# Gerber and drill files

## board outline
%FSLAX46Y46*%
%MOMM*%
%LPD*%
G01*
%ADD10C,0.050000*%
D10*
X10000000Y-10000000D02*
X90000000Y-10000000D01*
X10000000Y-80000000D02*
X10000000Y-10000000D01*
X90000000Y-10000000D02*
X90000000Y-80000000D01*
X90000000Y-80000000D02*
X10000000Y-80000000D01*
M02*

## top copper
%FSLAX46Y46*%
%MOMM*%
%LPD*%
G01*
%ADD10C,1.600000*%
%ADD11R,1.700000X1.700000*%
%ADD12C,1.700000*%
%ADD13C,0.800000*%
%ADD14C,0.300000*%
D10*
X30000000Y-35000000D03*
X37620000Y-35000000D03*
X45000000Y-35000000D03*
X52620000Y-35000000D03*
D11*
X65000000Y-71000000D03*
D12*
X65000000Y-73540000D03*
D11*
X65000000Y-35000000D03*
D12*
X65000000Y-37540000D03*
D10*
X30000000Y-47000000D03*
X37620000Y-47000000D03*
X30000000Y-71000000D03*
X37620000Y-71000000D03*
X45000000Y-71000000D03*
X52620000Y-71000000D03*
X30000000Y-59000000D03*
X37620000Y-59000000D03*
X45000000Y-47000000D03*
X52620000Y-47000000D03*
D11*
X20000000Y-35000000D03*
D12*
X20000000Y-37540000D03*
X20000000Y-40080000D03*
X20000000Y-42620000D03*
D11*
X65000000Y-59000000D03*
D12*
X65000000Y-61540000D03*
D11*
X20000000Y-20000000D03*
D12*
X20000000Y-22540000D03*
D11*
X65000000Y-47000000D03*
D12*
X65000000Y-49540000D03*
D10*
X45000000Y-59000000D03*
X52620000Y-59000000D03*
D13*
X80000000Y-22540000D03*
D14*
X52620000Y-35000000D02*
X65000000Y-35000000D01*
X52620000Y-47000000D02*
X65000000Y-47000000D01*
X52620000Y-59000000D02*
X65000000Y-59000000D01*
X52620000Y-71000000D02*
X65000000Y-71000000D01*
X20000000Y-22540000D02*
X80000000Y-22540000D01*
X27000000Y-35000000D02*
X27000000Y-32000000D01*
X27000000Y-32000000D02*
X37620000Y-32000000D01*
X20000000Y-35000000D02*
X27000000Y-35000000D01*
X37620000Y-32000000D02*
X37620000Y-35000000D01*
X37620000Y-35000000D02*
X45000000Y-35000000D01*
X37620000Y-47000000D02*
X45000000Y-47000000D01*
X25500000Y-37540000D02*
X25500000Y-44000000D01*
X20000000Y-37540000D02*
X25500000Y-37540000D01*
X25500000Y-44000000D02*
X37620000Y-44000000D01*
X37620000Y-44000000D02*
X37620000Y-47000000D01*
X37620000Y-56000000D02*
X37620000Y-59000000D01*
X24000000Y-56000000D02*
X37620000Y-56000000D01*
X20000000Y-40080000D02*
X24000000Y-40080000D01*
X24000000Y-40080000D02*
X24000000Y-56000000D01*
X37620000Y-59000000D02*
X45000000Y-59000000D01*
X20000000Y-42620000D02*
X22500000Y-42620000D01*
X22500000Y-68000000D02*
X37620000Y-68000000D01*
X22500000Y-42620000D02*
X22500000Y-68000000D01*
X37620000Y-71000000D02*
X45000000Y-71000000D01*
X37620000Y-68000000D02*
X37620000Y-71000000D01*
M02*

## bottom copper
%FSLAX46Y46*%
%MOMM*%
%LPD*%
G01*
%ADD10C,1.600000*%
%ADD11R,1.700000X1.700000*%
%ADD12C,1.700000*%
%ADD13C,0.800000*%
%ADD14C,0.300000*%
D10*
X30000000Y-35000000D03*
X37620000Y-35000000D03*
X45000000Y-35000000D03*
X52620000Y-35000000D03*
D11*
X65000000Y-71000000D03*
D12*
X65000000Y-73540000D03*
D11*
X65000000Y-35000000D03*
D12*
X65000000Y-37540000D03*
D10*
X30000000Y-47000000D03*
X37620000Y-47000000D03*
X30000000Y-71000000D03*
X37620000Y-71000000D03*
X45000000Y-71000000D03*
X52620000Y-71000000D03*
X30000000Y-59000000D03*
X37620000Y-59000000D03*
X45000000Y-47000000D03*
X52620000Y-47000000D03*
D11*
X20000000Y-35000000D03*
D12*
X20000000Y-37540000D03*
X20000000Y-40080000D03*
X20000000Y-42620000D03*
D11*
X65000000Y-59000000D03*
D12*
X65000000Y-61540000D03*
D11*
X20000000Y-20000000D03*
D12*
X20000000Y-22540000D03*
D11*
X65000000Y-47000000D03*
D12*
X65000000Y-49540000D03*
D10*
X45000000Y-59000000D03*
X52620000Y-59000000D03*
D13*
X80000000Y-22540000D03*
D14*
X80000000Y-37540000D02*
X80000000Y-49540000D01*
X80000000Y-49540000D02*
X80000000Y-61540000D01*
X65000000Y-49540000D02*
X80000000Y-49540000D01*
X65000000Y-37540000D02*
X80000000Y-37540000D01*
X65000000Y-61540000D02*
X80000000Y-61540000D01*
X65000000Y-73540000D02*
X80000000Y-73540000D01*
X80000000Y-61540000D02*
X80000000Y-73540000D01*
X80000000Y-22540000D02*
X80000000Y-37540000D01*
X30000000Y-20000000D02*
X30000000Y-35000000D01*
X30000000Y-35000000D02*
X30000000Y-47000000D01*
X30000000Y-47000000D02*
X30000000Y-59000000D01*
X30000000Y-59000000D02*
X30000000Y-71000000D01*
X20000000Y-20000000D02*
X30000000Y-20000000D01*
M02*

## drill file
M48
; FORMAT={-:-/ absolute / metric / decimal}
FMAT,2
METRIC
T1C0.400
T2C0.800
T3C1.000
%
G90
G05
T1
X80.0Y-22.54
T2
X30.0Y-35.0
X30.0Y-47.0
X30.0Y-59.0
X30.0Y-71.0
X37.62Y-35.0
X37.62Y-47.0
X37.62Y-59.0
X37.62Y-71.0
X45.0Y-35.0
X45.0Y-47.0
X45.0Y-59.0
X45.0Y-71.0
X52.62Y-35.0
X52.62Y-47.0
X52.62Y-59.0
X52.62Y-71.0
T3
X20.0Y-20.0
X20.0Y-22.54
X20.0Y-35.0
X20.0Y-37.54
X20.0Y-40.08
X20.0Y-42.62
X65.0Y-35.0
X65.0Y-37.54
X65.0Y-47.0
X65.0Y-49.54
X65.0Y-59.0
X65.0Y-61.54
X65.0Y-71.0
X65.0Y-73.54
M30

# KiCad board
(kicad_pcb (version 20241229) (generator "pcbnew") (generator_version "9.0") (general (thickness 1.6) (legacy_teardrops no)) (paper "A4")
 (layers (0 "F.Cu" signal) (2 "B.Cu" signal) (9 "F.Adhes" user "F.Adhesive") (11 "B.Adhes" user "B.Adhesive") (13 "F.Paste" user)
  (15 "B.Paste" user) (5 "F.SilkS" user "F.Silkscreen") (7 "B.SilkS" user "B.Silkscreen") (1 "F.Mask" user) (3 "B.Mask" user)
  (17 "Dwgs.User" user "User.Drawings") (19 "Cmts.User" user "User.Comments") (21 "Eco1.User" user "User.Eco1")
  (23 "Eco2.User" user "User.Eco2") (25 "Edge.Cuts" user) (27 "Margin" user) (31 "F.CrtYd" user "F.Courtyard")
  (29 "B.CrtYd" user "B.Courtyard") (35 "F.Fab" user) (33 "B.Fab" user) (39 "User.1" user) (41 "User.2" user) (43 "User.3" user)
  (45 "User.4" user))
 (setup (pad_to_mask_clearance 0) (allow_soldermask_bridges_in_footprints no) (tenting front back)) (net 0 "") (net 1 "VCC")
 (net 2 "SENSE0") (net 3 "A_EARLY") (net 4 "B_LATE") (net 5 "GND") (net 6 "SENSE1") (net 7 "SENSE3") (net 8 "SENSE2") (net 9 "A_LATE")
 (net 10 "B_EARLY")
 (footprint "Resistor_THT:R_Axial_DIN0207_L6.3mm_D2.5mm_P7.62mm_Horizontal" (layer "F.Cu") (at 30 35)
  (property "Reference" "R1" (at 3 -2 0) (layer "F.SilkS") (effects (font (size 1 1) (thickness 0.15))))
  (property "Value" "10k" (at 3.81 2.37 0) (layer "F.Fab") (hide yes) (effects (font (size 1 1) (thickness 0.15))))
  (pad "1" thru_hole circle (at 0 0) (size 1.6 1.6) (drill 0.8) (layers "*.Cu" "*.Mask") (remove_unused_layers no) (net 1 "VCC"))
  (pad "2" thru_hole circle (at 7.62 0) (size 1.6 1.6) (drill 0.8) (layers "*.Cu" "*.Mask") (remove_unused_layers no) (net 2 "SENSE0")))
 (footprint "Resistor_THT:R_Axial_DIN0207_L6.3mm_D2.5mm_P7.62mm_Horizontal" (layer "F.Cu") (at 45 35)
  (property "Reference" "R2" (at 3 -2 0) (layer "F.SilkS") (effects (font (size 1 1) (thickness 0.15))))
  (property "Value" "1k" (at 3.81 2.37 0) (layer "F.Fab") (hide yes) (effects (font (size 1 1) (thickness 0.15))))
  (pad "1" thru_hole circle (at 0 0) (size 1.6 1.6) (drill 0.8) (layers "*.Cu" "*.Mask") (remove_unused_layers no) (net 2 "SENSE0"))
  (pad "2" thru_hole circle (at 7.62 0) (size 1.6 1.6) (drill 0.8) (layers "*.Cu" "*.Mask") (remove_unused_layers no) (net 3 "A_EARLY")))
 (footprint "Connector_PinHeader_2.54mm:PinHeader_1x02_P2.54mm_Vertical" (layer "F.Cu") (at 65 71)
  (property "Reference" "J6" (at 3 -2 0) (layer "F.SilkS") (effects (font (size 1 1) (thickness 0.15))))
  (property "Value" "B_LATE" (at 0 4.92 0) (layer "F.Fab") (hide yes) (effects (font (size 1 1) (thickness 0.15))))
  (pad "1" thru_hole rect (at 0 0) (size 1.7 1.7) (drill 1) (layers "*.Cu" "*.Mask") (remove_unused_layers no) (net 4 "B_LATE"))
  (pad "2" thru_hole circle (at 0 2.54) (size 1.7 1.7) (drill 1) (layers "*.Cu" "*.Mask") (remove_unused_layers no) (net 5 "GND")))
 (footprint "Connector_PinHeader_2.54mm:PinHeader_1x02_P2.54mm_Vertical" (layer "F.Cu") (at 65 35)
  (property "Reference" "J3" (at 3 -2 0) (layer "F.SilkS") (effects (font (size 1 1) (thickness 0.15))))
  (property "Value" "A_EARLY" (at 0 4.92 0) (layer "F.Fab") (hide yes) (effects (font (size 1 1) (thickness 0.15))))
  (pad "1" thru_hole rect (at 0 0) (size 1.7 1.7) (drill 1) (layers "*.Cu" "*.Mask") (remove_unused_layers no) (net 3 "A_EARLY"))
  (pad "2" thru_hole circle (at 0 2.54) (size 1.7 1.7) (drill 1) (layers "*.Cu" "*.Mask") (remove_unused_layers no) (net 5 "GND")))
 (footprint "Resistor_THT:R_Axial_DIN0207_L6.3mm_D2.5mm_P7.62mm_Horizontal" (layer "F.Cu") (at 30 47)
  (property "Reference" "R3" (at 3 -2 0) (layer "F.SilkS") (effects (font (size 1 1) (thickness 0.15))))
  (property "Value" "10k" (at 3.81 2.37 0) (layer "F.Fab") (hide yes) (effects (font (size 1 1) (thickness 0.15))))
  (pad "1" thru_hole circle (at 0 0) (size 1.6 1.6) (drill 0.8) (layers "*.Cu" "*.Mask") (remove_unused_layers no) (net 1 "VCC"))
  (pad "2" thru_hole circle (at 7.62 0) (size 1.6 1.6) (drill 0.8) (layers "*.Cu" "*.Mask") (remove_unused_layers no) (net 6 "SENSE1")))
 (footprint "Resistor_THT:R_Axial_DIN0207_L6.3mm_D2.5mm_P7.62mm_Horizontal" (layer "F.Cu") (at 30 71)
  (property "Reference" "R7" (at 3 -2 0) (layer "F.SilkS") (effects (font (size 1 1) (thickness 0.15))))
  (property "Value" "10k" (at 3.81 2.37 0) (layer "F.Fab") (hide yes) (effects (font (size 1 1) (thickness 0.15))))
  (pad "1" thru_hole circle (at 0 0) (size 1.6 1.6) (drill 0.8) (layers "*.Cu" "*.Mask") (remove_unused_layers no) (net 1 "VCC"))
  (pad "2" thru_hole circle (at 7.62 0) (size 1.6 1.6) (drill 0.8) (layers "*.Cu" "*.Mask") (remove_unused_layers no) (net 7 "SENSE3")))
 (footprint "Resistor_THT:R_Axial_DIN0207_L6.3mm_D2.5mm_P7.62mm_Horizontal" (layer "F.Cu") (at 45 71)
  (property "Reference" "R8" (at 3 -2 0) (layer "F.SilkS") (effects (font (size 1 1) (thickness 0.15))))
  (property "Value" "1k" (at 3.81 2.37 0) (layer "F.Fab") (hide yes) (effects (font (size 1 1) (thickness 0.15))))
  (pad "1" thru_hole circle (at 0 0) (size 1.6 1.6) (drill 0.8) (layers "*.Cu" "*.Mask") (remove_unused_layers no) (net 7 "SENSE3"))
  (pad "2" thru_hole circle (at 7.62 0) (size 1.6 1.6) (drill 0.8) (layers "*.Cu" "*.Mask") (remove_unused_layers no) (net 4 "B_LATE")))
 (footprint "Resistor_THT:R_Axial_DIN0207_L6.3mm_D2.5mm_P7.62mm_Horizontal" (layer "F.Cu") (at 30 59)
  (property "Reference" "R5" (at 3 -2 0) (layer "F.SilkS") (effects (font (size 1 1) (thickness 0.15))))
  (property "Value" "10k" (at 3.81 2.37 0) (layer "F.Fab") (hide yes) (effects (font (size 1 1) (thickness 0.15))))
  (pad "1" thru_hole circle (at 0 0) (size 1.6 1.6) (drill 0.8) (layers "*.Cu" "*.Mask") (remove_unused_layers no) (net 1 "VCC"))
  (pad "2" thru_hole circle (at 7.62 0) (size 1.6 1.6) (drill 0.8) (layers "*.Cu" "*.Mask") (remove_unused_layers no) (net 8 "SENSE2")))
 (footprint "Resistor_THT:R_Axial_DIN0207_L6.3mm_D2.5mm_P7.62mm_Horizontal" (layer "F.Cu") (at 45 47)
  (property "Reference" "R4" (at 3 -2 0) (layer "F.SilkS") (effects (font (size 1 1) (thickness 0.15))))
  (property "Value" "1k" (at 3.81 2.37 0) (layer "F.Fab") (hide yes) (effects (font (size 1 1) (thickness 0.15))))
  (pad "1" thru_hole circle (at 0 0) (size 1.6 1.6) (drill 0.8) (layers "*.Cu" "*.Mask") (remove_unused_layers no) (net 6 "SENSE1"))
  (pad "2" thru_hole circle (at 7.62 0) (size 1.6 1.6) (drill 0.8) (layers "*.Cu" "*.Mask") (remove_unused_layers no) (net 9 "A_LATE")))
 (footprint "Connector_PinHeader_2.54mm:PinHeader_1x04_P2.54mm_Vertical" (layer "F.Cu") (at 20 35)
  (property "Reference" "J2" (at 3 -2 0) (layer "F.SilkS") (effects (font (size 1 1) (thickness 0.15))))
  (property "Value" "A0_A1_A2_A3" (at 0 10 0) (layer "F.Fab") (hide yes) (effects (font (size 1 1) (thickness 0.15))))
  (pad "1" thru_hole rect (at 0 0) (size 1.7 1.7) (drill 1) (layers "*.Cu" "*.Mask") (remove_unused_layers no) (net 2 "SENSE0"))
  (pad "2" thru_hole circle (at 0 2.54) (size 1.7 1.7) (drill 1) (layers "*.Cu" "*.Mask") (remove_unused_layers no) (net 6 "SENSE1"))
  (pad "3" thru_hole circle (at 0 5.08) (size 1.7 1.7) (drill 1) (layers "*.Cu" "*.Mask") (remove_unused_layers no) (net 8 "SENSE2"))
  (pad "4" thru_hole circle (at 0 7.62) (size 1.7 1.7) (drill 1) (layers "*.Cu" "*.Mask") (remove_unused_layers no) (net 7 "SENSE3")))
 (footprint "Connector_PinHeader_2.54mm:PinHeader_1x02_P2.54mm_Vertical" (layer "F.Cu") (at 65 59)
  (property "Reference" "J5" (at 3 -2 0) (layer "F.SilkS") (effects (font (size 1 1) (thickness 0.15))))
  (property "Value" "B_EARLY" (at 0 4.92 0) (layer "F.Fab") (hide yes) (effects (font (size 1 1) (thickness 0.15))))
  (pad "1" thru_hole rect (at 0 0) (size 1.7 1.7) (drill 1) (layers "*.Cu" "*.Mask") (remove_unused_layers no) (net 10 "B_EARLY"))
  (pad "2" thru_hole circle (at 0 2.54) (size 1.7 1.7) (drill 1) (layers "*.Cu" "*.Mask") (remove_unused_layers no) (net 5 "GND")))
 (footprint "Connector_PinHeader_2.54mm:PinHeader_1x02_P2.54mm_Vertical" (layer "F.Cu") (at 20 20)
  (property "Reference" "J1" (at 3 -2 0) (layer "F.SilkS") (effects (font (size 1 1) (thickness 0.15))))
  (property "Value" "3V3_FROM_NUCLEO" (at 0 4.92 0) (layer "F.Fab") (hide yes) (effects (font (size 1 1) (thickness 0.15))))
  (pad "1" thru_hole rect (at 0 0) (size 1.7 1.7) (drill 1) (layers "*.Cu" "*.Mask") (remove_unused_layers no) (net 1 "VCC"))
  (pad "2" thru_hole circle (at 0 2.54) (size 1.7 1.7) (drill 1) (layers "*.Cu" "*.Mask") (remove_unused_layers no) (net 5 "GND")))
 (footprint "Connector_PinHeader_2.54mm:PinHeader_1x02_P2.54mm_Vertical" (layer "F.Cu") (at 65 47)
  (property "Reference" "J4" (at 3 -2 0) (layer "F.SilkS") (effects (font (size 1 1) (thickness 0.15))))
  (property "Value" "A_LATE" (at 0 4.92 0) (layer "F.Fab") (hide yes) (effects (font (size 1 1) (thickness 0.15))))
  (pad "1" thru_hole rect (at 0 0) (size 1.7 1.7) (drill 1) (layers "*.Cu" "*.Mask") (remove_unused_layers no) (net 9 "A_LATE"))
  (pad "2" thru_hole circle (at 0 2.54) (size 1.7 1.7) (drill 1) (layers "*.Cu" "*.Mask") (remove_unused_layers no) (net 5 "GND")))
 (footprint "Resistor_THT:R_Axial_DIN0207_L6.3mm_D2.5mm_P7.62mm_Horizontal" (layer "F.Cu") (at 45 59)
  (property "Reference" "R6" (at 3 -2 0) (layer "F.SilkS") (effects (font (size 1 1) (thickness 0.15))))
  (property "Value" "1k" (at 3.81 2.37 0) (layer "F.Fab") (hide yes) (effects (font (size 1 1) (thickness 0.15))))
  (pad "1" thru_hole circle (at 0 0) (size 1.6 1.6) (drill 0.8) (layers "*.Cu" "*.Mask") (remove_unused_layers no) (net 8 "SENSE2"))
  (pad "2" thru_hole circle (at 7.62 0) (size 1.6 1.6) (drill 0.8) (layers "*.Cu" "*.Mask") (remove_unused_layers no) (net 10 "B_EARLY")))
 (gr_line (start 10 10) (end 90 10) (stroke (width 0.05) (type default)) (layer "Edge.Cuts"))
 (gr_line (start 10 80) (end 10 10) (stroke (width 0.05) (type default)) (layer "Edge.Cuts"))
 (gr_line (start 90 10) (end 90 80) (stroke (width 0.05) (type default)) (layer "Edge.Cuts"))
 (gr_line (start 90 80) (end 10 80) (stroke (width 0.05) (type default)) (layer "Edge.Cuts"))
 (segment (start 52.62 35) (end 65 35) (width 0.3) (layer "F.Cu") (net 3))
 (segment (start 52.62 47) (end 65 47) (width 0.3) (layer "F.Cu") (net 9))
 (segment (start 52.62 59) (end 65 59) (width 0.3) (layer "F.Cu") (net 10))
 (segment (start 52.62 71) (end 65 71) (width 0.3) (layer "F.Cu") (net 4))
 (segment (start 20 22.54) (end 80 22.54) (width 0.3) (layer "F.Cu") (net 5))
 (via (at 80 22.54) (size 0.8) (drill 0.4) (layers "F.Cu" "B.Cu") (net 5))
 (segment (start 80 37.54) (end 80 49.54) (width 0.3) (layer "B.Cu") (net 5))
 (segment (start 80 49.54) (end 80 61.54) (width 0.3) (layer "B.Cu") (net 5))
 (segment (start 65 49.54) (end 80 49.54) (width 0.3) (layer "B.Cu") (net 5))
 (segment (start 65 37.54) (end 80 37.54) (width 0.3) (layer "B.Cu") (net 5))
 (segment (start 65 61.54) (end 80 61.54) (width 0.3) (layer "B.Cu") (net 5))
 (segment (start 65 73.54) (end 80 73.54) (width 0.3) (layer "B.Cu") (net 5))
 (segment (start 80 61.54) (end 80 73.54) (width 0.3) (layer "B.Cu") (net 5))
 (segment (start 80 22.54) (end 80 37.54) (width 0.3) (layer "B.Cu") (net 5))
 (segment (start 27 35) (end 27 32) (width 0.3) (layer "F.Cu") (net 2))
 (segment (start 27 32) (end 37.62 32) (width 0.3) (layer "F.Cu") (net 2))
 (segment (start 20 35) (end 27 35) (width 0.3) (layer "F.Cu") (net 2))
 (segment (start 37.62 32) (end 37.62 35) (width 0.3) (layer "F.Cu") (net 2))
 (segment (start 37.62 35) (end 45 35) (width 0.3) (layer "F.Cu") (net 2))
 (segment (start 37.62 47) (end 45 47) (width 0.3) (layer "F.Cu") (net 6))
 (segment (start 25.5 37.54) (end 25.5 44) (width 0.3) (layer "F.Cu") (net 6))
 (segment (start 20 37.54) (end 25.5 37.54) (width 0.3) (layer "F.Cu") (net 6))
 (segment (start 25.5 44) (end 37.62 44) (width 0.3) (layer "F.Cu") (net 6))
 (segment (start 37.62 44) (end 37.62 47) (width 0.3) (layer "F.Cu") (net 6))
 (segment (start 37.62 56) (end 37.62 59) (width 0.3) (layer "F.Cu") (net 8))
 (segment (start 24 56) (end 37.62 56) (width 0.3) (layer "F.Cu") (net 8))
 (segment (start 20 40.08) (end 24 40.08) (width 0.3) (layer "F.Cu") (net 8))
 (segment (start 24 40.08) (end 24 56) (width 0.3) (layer "F.Cu") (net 8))
 (segment (start 37.62 59) (end 45 59) (width 0.3) (layer "F.Cu") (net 8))
 (segment (start 20 42.62) (end 22.5 42.62) (width 0.3) (layer "F.Cu") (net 7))
 (segment (start 22.5 68) (end 37.62 68) (width 0.3) (layer "F.Cu") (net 7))
 (segment (start 22.5 42.62) (end 22.5 68) (width 0.3) (layer "F.Cu") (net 7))
 (segment (start 37.62 71) (end 45 71) (width 0.3) (layer "F.Cu") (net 7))
 (segment (start 37.62 68) (end 37.62 71) (width 0.3) (layer "F.Cu") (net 7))
 (segment (start 30 20) (end 30 35) (width 0.3) (layer "B.Cu") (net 1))
 (segment (start 30 35) (end 30 47) (width 0.3) (layer "B.Cu") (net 1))
 (segment (start 30 47) (end 30 59) (width 0.3) (layer "B.Cu") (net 1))
 (segment (start 30 59) (end 30 71) (width 0.3) (layer "B.Cu") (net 1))
 (segment (start 20 20) (end 30 20) (width 0.3) (layer "B.Cu") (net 1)))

